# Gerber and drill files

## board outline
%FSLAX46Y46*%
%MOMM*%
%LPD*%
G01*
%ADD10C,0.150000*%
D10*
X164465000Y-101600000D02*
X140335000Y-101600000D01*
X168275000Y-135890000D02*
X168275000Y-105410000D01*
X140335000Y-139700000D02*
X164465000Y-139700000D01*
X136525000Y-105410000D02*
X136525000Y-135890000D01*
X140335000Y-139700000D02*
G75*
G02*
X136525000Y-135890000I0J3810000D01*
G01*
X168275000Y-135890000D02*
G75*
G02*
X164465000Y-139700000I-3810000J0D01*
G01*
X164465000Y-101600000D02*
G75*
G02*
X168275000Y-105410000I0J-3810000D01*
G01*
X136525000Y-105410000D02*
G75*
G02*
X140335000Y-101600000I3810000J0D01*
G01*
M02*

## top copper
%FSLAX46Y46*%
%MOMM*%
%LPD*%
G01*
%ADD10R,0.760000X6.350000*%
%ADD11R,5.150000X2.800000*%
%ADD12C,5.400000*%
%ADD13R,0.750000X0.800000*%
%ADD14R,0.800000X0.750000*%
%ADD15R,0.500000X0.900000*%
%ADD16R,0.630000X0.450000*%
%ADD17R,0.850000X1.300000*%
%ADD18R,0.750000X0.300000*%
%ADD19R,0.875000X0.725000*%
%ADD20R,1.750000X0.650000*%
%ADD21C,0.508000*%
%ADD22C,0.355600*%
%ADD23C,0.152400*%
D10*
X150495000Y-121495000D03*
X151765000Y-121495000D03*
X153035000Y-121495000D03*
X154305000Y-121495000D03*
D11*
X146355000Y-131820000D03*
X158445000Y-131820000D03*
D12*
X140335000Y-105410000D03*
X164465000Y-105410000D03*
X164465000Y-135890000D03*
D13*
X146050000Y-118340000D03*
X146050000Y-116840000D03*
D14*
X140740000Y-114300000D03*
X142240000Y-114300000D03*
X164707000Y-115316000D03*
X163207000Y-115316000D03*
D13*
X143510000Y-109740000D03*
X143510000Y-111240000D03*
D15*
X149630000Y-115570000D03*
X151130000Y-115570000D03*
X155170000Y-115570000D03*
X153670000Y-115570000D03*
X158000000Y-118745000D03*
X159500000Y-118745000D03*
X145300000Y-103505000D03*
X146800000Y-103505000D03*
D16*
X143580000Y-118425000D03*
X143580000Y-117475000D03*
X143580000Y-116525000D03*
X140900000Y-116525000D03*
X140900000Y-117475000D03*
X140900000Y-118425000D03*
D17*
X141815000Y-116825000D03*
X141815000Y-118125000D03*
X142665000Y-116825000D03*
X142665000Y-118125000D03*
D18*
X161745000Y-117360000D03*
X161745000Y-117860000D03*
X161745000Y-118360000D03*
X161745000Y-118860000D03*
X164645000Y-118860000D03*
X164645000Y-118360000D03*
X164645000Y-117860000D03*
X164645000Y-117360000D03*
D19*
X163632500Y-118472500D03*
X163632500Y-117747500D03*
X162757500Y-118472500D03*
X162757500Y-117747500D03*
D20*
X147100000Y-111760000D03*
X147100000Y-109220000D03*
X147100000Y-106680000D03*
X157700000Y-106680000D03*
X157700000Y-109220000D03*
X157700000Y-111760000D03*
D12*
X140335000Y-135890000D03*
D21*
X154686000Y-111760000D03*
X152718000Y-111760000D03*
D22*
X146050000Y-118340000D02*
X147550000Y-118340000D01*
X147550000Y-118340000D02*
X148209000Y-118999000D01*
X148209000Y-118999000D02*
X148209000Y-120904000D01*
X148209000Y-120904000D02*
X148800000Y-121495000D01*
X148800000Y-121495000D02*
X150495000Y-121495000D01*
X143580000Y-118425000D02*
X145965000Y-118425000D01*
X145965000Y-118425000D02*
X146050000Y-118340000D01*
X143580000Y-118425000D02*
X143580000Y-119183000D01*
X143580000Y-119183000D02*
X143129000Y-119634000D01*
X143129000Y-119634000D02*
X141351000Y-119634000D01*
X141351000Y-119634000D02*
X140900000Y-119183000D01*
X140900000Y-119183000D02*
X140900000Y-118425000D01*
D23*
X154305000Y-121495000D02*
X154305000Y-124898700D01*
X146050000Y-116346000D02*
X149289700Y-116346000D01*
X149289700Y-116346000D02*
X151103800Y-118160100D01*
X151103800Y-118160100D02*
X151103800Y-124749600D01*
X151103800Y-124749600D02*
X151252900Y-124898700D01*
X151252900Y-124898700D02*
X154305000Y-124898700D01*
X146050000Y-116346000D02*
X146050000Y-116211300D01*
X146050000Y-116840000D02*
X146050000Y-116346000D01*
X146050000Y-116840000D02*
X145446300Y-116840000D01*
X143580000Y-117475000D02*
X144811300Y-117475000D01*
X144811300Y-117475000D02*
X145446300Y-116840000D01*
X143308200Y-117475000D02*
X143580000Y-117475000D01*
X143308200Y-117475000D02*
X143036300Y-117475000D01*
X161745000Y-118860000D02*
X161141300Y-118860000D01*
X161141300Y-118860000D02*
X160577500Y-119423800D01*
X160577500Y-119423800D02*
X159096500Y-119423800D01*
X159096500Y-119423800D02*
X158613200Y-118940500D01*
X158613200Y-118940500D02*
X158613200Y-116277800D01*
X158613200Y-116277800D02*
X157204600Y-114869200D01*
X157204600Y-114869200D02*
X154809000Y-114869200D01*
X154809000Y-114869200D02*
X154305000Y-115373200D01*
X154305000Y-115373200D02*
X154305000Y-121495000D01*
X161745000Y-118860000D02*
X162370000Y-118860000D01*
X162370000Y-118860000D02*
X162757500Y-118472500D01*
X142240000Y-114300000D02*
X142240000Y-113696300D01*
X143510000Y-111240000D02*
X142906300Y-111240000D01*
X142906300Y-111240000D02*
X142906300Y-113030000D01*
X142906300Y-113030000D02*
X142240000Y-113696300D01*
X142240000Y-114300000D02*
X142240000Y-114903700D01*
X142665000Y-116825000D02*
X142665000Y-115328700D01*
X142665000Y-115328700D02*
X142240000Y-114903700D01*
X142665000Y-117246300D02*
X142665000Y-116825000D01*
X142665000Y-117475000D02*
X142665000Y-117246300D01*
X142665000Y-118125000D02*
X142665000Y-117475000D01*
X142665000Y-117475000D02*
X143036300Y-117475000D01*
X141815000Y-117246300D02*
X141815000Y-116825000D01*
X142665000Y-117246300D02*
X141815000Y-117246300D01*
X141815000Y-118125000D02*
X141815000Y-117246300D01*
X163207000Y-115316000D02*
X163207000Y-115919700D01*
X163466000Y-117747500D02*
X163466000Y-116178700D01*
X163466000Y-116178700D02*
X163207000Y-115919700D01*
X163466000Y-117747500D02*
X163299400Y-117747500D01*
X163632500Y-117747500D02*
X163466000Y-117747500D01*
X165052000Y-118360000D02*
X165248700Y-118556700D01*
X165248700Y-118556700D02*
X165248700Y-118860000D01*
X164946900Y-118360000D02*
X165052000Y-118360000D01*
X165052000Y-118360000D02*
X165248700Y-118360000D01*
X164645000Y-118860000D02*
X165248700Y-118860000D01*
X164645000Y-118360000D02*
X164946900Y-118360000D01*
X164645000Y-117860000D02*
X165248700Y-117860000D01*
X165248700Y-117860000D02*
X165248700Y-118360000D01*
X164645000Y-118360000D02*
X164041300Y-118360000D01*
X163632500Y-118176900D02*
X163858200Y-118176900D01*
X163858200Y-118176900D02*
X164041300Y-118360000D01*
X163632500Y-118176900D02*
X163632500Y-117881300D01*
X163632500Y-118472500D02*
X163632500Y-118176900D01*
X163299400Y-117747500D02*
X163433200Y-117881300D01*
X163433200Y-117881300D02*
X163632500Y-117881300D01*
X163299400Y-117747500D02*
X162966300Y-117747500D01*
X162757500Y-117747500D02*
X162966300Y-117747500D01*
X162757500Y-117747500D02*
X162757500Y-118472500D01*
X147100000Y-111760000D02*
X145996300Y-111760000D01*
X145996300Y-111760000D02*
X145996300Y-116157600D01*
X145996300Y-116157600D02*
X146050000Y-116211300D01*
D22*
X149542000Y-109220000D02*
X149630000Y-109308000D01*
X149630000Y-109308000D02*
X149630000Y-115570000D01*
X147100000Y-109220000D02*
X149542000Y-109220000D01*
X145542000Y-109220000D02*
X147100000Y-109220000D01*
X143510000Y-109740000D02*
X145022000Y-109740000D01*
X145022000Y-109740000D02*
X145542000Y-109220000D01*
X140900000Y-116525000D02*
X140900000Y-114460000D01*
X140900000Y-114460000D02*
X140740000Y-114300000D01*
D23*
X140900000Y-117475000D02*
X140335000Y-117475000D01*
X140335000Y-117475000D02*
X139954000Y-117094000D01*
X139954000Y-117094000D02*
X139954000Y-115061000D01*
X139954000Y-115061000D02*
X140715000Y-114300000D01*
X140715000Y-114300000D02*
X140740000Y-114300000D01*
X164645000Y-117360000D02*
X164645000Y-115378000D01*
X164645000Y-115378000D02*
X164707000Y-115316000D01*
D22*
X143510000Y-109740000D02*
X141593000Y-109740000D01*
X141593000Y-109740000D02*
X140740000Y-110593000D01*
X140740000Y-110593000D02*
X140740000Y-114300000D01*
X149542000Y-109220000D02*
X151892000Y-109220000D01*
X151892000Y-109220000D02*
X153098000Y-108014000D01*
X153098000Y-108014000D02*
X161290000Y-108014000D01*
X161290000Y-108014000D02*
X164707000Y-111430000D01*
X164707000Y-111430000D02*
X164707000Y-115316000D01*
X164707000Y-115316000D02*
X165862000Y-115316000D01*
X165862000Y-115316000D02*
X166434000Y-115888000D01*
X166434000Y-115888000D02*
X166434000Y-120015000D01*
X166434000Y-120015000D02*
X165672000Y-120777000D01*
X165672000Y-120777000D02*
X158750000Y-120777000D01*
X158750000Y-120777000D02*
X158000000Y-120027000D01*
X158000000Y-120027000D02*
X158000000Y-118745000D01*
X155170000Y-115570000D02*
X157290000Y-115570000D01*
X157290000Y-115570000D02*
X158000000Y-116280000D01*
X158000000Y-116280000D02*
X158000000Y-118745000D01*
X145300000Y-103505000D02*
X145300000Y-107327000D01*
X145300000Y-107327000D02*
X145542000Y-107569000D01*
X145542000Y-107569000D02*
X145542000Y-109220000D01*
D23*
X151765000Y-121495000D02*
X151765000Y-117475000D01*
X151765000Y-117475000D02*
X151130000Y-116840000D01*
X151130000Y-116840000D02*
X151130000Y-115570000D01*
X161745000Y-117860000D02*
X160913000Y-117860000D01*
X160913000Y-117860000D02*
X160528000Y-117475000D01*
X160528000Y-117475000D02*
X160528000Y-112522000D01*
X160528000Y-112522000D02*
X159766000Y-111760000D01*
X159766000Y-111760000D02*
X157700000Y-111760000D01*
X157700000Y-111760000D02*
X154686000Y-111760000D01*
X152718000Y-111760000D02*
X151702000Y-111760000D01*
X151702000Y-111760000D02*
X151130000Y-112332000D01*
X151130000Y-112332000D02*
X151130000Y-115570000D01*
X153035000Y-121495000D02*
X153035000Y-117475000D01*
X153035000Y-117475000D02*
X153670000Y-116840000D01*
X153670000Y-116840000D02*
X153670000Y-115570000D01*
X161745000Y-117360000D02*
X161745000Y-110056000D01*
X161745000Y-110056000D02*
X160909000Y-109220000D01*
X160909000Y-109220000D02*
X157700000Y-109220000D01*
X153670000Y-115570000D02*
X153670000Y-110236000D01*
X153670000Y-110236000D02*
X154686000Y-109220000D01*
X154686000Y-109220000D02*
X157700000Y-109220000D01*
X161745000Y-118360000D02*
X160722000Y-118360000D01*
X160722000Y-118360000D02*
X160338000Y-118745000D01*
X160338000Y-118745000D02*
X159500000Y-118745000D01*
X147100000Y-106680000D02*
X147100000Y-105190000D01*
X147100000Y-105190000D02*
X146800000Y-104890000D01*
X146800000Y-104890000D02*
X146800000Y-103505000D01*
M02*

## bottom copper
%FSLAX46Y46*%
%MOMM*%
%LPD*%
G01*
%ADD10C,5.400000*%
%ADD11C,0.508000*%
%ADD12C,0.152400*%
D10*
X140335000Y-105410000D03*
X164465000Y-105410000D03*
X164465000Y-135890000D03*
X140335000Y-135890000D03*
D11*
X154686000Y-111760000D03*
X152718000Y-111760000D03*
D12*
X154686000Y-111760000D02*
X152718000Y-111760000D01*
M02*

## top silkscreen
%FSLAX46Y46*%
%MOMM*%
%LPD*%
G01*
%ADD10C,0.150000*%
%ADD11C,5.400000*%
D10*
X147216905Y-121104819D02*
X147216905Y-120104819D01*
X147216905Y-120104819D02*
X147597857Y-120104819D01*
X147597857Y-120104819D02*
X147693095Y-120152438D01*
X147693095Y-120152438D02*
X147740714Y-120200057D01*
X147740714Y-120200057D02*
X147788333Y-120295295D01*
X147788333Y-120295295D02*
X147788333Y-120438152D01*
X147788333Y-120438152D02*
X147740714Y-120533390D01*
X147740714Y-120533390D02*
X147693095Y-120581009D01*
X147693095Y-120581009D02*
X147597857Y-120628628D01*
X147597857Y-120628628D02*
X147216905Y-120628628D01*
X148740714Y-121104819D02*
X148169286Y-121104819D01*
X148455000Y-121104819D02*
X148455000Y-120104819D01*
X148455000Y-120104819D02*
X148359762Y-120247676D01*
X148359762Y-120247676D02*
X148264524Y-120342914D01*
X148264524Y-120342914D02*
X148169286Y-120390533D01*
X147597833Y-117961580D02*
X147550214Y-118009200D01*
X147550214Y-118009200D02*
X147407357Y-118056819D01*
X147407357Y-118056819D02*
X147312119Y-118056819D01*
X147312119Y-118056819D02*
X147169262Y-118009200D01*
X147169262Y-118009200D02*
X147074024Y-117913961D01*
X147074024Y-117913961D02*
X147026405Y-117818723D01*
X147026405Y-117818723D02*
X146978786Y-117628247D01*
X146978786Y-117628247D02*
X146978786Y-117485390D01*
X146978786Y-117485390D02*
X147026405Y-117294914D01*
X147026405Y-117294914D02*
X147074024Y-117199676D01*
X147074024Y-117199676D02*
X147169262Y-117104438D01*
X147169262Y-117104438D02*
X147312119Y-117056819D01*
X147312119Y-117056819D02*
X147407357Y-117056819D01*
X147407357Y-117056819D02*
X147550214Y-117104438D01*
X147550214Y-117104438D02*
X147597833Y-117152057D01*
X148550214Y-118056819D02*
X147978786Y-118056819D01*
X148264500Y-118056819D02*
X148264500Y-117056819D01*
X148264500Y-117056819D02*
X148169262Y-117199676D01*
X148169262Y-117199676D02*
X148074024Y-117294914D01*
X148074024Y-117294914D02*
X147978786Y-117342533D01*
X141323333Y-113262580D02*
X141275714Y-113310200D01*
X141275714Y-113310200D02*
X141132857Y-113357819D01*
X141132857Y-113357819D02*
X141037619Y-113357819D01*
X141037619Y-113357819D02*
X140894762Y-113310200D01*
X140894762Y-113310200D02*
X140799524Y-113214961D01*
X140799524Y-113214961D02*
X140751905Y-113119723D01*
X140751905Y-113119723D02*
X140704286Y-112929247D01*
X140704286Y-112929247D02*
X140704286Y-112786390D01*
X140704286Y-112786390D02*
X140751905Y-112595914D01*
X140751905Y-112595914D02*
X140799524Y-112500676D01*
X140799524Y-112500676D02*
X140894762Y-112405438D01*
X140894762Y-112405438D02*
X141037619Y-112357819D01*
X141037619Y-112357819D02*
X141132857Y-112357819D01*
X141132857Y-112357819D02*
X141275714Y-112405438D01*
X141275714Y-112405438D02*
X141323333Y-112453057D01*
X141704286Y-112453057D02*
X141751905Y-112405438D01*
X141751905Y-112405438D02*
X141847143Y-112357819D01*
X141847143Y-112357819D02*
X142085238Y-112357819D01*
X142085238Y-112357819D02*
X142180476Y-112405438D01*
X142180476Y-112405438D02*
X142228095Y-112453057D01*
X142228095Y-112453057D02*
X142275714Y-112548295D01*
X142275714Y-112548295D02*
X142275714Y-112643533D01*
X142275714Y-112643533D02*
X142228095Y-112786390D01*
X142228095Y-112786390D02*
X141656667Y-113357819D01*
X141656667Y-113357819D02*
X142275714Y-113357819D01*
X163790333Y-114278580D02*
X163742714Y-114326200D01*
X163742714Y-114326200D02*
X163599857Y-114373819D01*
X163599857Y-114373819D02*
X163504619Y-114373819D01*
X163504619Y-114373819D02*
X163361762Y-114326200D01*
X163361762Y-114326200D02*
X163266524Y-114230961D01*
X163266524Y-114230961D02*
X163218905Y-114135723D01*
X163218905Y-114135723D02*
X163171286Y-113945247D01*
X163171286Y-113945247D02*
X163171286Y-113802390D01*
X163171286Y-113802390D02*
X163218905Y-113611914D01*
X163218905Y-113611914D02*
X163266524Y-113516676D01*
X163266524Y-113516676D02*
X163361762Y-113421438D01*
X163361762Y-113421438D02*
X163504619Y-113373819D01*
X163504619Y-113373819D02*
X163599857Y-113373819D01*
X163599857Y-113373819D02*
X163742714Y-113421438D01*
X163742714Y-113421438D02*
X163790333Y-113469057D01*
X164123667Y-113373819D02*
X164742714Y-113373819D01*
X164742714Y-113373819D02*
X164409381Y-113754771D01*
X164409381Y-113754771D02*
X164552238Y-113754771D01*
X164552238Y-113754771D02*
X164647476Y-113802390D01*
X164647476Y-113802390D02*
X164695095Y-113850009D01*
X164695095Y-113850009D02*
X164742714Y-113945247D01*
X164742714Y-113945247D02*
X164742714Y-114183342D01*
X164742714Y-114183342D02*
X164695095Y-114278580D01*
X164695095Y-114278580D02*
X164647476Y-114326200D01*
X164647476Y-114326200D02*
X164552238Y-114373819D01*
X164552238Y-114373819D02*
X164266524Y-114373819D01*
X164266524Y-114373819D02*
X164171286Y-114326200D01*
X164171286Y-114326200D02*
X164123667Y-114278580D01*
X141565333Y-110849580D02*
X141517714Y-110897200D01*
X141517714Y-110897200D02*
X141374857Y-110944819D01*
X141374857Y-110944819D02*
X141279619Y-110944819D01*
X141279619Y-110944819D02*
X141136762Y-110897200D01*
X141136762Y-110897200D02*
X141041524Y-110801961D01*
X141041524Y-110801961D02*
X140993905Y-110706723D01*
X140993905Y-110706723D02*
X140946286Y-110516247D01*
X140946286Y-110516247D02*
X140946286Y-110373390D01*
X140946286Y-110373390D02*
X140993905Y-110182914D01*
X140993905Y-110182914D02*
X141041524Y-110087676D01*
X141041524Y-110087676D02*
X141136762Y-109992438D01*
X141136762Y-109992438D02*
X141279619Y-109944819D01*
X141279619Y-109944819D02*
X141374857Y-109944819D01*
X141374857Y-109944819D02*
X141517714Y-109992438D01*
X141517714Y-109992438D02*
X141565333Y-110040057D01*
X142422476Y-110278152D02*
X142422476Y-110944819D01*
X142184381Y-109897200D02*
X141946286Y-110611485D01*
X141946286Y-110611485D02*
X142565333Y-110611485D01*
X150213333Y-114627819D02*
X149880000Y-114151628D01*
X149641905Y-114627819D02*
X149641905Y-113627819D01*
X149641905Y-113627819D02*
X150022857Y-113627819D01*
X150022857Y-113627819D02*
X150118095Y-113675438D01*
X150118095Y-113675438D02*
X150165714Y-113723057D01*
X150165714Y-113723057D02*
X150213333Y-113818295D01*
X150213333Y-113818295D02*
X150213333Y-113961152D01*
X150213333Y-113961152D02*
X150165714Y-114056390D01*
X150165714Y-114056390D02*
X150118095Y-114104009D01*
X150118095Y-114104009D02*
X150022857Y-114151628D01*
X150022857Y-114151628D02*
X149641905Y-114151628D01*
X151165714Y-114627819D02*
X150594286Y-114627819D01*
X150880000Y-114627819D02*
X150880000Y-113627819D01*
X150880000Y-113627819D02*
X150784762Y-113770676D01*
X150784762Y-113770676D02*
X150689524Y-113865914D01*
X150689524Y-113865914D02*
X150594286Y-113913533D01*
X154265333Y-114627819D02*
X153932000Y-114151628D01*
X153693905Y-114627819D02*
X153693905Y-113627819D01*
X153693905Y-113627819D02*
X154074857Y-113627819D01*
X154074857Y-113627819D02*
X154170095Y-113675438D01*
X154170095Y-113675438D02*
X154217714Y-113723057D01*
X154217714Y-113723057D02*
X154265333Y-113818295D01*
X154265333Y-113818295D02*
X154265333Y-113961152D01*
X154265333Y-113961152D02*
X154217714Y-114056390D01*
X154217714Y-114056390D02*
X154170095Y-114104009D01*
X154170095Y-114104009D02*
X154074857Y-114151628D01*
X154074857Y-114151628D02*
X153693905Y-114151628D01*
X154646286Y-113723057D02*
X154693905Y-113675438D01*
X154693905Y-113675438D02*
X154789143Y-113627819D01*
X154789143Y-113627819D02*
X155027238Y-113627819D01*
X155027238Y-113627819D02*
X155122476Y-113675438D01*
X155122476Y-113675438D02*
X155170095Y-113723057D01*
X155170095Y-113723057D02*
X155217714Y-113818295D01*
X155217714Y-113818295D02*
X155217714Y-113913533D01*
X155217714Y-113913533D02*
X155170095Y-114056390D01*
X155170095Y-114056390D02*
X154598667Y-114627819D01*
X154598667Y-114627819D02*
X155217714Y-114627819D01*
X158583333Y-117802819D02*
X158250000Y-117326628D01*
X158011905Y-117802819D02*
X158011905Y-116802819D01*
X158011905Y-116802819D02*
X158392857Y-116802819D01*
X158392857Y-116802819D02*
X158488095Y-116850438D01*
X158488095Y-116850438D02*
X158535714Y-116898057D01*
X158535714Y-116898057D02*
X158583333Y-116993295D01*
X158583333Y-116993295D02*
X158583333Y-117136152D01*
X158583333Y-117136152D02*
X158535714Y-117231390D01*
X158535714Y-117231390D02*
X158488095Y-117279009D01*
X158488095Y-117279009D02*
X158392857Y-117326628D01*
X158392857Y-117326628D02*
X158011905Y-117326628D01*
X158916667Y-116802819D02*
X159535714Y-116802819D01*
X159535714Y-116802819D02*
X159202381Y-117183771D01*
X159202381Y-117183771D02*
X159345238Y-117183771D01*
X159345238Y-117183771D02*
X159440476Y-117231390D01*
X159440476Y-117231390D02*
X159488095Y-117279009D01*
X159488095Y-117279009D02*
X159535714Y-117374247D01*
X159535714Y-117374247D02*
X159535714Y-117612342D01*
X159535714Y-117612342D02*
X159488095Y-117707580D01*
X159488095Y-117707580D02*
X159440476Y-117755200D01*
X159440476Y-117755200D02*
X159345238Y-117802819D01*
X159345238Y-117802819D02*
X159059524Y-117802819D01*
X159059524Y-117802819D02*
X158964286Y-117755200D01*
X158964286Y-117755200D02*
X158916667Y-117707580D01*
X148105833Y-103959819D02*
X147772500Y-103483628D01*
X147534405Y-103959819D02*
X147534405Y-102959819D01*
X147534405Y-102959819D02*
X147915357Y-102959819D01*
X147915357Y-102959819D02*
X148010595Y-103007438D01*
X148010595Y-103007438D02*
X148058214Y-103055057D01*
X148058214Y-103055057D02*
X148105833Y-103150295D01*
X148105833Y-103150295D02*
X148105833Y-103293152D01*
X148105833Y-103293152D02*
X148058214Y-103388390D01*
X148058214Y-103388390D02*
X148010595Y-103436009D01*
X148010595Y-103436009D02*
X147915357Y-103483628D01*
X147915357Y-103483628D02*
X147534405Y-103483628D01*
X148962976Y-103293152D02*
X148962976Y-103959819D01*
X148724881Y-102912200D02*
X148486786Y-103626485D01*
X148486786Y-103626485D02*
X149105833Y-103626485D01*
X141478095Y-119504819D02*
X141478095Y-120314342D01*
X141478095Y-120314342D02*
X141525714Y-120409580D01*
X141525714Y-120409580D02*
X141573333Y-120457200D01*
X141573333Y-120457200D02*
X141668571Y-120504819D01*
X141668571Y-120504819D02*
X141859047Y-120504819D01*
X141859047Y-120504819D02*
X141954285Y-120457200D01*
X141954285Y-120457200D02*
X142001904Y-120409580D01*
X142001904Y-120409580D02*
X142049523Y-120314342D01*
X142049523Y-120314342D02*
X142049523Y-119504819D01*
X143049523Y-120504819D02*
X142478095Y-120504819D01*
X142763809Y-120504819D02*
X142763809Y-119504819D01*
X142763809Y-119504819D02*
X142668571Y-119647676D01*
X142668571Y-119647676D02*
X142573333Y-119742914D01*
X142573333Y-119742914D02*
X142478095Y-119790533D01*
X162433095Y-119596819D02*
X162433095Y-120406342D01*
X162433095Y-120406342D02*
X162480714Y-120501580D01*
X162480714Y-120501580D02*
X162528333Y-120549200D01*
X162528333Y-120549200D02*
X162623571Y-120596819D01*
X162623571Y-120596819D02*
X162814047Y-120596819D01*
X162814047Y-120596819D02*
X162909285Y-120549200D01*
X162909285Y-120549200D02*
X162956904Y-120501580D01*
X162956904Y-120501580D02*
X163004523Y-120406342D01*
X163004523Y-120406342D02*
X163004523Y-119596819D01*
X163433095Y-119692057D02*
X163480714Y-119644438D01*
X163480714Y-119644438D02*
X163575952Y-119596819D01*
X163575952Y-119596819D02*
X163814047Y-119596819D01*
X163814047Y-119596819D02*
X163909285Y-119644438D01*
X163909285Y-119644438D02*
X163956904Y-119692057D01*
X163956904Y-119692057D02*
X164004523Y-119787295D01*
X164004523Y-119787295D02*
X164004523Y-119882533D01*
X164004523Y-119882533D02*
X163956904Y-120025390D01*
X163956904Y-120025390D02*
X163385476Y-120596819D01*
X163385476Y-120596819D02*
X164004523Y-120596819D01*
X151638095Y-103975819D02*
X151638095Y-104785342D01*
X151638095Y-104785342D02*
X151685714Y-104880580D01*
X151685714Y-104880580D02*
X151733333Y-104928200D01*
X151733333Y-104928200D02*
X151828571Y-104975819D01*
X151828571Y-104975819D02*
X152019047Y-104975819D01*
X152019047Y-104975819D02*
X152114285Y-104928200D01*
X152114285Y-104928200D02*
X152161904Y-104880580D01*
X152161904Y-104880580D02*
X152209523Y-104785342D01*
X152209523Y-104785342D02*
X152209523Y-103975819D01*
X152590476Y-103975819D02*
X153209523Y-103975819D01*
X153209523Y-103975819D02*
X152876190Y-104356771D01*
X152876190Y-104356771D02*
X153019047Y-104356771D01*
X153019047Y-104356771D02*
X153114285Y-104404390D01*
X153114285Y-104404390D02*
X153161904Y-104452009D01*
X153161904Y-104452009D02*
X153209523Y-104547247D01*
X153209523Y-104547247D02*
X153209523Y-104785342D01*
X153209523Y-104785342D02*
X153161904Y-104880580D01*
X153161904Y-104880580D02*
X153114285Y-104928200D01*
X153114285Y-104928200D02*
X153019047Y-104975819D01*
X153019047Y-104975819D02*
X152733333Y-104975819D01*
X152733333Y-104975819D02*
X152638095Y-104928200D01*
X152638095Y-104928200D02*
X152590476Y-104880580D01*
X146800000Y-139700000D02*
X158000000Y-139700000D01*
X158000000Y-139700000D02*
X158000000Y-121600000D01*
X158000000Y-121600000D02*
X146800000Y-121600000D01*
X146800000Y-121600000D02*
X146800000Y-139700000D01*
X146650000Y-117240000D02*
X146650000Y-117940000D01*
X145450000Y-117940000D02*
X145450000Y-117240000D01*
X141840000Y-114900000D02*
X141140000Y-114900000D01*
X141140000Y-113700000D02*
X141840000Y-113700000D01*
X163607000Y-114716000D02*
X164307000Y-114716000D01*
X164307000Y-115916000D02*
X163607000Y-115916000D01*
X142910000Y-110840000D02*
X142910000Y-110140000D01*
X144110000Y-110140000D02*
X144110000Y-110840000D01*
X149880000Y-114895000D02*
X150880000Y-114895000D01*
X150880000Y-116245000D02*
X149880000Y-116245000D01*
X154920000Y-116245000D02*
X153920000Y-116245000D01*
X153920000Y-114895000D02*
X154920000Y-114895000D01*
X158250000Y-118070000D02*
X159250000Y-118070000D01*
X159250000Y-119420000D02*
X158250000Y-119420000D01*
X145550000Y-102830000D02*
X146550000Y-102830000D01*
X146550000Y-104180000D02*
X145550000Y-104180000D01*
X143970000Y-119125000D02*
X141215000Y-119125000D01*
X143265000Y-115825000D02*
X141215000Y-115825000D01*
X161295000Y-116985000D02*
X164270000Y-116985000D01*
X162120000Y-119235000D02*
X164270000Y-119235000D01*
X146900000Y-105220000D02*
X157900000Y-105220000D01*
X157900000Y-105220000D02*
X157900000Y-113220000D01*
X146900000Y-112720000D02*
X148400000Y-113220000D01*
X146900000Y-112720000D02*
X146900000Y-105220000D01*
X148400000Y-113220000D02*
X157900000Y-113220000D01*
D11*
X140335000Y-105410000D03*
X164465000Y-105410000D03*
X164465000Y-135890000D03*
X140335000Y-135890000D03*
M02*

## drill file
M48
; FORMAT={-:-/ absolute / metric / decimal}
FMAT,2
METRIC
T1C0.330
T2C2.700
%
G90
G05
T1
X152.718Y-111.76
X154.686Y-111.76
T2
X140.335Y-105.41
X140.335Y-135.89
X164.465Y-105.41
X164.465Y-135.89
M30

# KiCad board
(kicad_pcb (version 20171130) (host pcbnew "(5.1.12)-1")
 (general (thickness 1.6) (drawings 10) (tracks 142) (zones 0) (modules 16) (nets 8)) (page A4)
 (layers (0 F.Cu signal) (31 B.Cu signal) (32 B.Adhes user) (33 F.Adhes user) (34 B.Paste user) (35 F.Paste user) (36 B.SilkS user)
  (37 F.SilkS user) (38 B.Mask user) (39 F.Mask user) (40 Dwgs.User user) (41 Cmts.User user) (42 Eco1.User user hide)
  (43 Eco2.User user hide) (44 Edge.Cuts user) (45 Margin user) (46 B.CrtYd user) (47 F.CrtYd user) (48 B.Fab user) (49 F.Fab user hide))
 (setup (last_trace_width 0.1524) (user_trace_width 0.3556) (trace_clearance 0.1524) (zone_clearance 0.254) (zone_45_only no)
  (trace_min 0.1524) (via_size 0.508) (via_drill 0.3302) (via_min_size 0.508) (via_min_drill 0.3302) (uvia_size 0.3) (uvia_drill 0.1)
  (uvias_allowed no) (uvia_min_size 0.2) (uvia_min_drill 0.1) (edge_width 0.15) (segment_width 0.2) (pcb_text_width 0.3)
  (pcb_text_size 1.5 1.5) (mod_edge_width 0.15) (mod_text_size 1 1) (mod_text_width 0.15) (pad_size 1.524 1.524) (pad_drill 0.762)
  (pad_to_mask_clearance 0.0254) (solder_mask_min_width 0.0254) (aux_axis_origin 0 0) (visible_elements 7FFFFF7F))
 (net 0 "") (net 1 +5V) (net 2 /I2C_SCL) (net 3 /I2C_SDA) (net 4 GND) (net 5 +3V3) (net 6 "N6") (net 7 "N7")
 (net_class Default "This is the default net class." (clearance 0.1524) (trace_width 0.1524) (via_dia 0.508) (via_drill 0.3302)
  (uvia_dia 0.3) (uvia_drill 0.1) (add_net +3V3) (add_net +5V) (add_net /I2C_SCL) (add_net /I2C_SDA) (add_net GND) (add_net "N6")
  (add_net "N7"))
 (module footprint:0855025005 (layer F.Cu) (at 152.4 139.7)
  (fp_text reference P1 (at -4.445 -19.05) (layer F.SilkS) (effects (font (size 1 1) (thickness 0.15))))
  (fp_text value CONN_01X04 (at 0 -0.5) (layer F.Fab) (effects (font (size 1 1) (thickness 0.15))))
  (fp_line (start -5.6 0) (end 5.6 0) (layer F.SilkS) (width 0.15))
  (fp_line (start 5.6 0) (end 5.6 -18.1) (layer F.SilkS) (width 0.15))
  (fp_line (start 5.6 -18.1) (end -5.6 -18.1) (layer F.SilkS) (width 0.15))
  (fp_line (start -5.6 -18.1) (end -5.6 0) (layer F.SilkS) (width 0.15))
  (pad 1 smd rect (at -1.905 -18.205) (size 0.76 6.35) (layers F.Cu F.Paste F.Mask) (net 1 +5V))
  (pad 2 smd rect (at -0.635 -18.205) (size 0.76 6.35) (layers F.Cu F.Paste F.Mask) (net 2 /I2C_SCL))
  (pad 3 smd rect (at 0.635 -18.205) (size 0.76 6.35) (layers F.Cu F.Paste F.Mask) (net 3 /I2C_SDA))
  (pad 4 smd rect (at 1.905 -18.205) (size 0.76 6.35) (layers F.Cu F.Paste F.Mask) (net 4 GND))
  (pad 5 smd rect (at -6.045 -7.88) (size 5.15 2.8) (layers F.Cu F.Paste F.Mask))
  (pad 5 smd rect (at 6.045 -7.88) (size 5.15 2.8) (layers F.Cu F.Paste F.Mask)))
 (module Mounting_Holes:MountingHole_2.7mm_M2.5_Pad (layer F.Cu) (at 140.335 105.41)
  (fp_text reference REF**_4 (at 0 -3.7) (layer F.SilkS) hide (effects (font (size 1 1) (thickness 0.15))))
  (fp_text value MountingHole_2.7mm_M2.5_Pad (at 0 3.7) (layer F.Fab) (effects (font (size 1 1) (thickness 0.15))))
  (pad 1 thru_hole circle (at 0 0) (size 5.4 5.4) (drill 2.7) (layers *.Cu *.Mask F.SilkS)))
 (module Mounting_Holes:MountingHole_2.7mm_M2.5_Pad (layer F.Cu) (at 164.465 105.41)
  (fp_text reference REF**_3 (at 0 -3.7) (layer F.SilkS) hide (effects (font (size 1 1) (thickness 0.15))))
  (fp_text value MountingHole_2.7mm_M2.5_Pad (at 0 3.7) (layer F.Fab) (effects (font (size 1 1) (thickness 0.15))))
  (pad 1 thru_hole circle (at 0 0) (size 5.4 5.4) (drill 2.7) (layers *.Cu *.Mask F.SilkS)))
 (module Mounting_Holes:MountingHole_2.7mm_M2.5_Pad (layer F.Cu) (at 164.465 135.89)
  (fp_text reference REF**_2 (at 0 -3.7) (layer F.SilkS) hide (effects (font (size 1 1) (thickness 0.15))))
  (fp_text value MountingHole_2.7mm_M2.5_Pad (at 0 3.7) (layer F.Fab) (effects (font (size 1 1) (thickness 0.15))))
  (pad 1 thru_hole circle (at 0 0) (size 5.4 5.4) (drill 2.7) (layers *.Cu *.Mask F.SilkS)))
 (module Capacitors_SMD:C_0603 (layer F.Cu) (at 146.05 117.59 90)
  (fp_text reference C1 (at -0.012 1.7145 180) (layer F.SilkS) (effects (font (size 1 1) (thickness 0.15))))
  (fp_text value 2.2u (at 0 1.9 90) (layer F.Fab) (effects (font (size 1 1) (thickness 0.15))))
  (fp_line (start 0.35 0.6) (end -0.35 0.6) (layer F.SilkS) (width 0.15))
  (fp_line (start -0.35 -0.6) (end 0.35 -0.6) (layer F.SilkS) (width 0.15))
  (pad 1 smd rect (at -0.75 0 90) (size 0.8 0.75) (layers F.Cu F.Paste F.Mask) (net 1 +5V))
  (pad 2 smd rect (at 0.75 0 90) (size 0.8 0.75) (layers F.Cu F.Paste F.Mask) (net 4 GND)))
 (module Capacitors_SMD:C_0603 (layer F.Cu) (at 141.49 114.3)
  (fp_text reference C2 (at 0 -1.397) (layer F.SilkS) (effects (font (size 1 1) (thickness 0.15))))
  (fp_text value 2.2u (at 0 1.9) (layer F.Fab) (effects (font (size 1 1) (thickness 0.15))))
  (fp_line (start 0.35 0.6) (end -0.35 0.6) (layer F.SilkS) (width 0.15))
  (fp_line (start -0.35 -0.6) (end 0.35 -0.6) (layer F.SilkS) (width 0.15))
  (pad 1 smd rect (at -0.75 0) (size 0.8 0.75) (layers F.Cu F.Paste F.Mask) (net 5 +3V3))
  (pad 2 smd rect (at 0.75 0) (size 0.8 0.75) (layers F.Cu F.Paste F.Mask) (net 4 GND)))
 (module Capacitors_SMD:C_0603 (layer F.Cu) (at 163.957 115.316 180)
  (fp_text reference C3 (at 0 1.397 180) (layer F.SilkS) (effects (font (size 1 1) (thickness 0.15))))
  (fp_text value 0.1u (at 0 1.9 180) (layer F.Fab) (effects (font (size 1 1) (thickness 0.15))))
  (fp_line (start 0.35 0.6) (end -0.35 0.6) (layer F.SilkS) (width 0.15))
  (fp_line (start -0.35 -0.6) (end 0.35 -0.6) (layer F.SilkS) (width 0.15))
  (pad 1 smd rect (at -0.75 0 180) (size 0.8 0.75) (layers F.Cu F.Paste F.Mask) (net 5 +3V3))
  (pad 2 smd rect (at 0.75 0 180) (size 0.8 0.75) (layers F.Cu F.Paste F.Mask) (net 4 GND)))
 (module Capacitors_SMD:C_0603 (layer F.Cu) (at 143.51 110.49 270)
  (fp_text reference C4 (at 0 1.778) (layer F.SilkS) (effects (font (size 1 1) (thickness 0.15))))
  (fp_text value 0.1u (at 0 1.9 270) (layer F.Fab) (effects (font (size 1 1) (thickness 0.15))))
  (fp_line (start 0.35 0.6) (end -0.35 0.6) (layer F.SilkS) (width 0.15))
  (fp_line (start -0.35 -0.6) (end 0.35 -0.6) (layer F.SilkS) (width 0.15))
  (pad 1 smd rect (at -0.75 0 270) (size 0.8 0.75) (layers F.Cu F.Paste F.Mask) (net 5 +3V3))
  (pad 2 smd rect (at 0.75 0 270) (size 0.8 0.75) (layers F.Cu F.Paste F.Mask) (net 4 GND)))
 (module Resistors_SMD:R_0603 (layer F.Cu) (at 150.38 115.57)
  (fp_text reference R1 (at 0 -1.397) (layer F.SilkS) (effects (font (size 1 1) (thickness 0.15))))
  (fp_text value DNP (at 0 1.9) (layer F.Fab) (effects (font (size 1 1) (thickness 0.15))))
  (fp_line (start -0.5 -0.675) (end 0.5 -0.675) (layer F.SilkS) (width 0.15))
  (fp_line (start 0.5 0.675) (end -0.5 0.675) (layer F.SilkS) (width 0.15))
  (pad 1 smd rect (at -0.75 0) (size 0.5 0.9) (layers F.Cu F.Paste F.Mask) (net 5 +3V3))
  (pad 2 smd rect (at 0.75 0) (size 0.5 0.9) (layers F.Cu F.Paste F.Mask) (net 2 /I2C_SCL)))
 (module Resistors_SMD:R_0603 (layer F.Cu) (at 154.42 115.57 180)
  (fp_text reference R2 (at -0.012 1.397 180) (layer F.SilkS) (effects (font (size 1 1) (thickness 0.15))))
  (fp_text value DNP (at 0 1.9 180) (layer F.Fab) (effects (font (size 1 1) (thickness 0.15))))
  (fp_line (start -0.5 -0.675) (end 0.5 -0.675) (layer F.SilkS) (width 0.15))
  (fp_line (start 0.5 0.675) (end -0.5 0.675) (layer F.SilkS) (width 0.15))
  (pad 1 smd rect (at -0.75 0 180) (size 0.5 0.9) (layers F.Cu F.Paste F.Mask) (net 5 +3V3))
  (pad 2 smd rect (at 0.75 0 180) (size 0.5 0.9) (layers F.Cu F.Paste F.Mask) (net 3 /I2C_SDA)))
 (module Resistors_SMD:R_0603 (layer F.Cu) (at 158.75 118.745)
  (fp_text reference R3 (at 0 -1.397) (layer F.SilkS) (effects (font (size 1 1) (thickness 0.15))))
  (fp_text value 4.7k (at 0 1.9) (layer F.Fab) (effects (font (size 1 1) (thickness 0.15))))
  (fp_line (start -0.5 -0.675) (end 0.5 -0.675) (layer F.SilkS) (width 0.15))
  (fp_line (start 0.5 0.675) (end -0.5 0.675) (layer F.SilkS) (width 0.15))
  (pad 1 smd rect (at -0.75 0) (size 0.5 0.9) (layers F.Cu F.Paste F.Mask) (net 5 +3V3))
  (pad 2 smd rect (at 0.75 0) (size 0.5 0.9) (layers F.Cu F.Paste F.Mask) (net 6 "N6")))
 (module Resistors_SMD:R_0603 (layer F.Cu) (at 146.05 103.505)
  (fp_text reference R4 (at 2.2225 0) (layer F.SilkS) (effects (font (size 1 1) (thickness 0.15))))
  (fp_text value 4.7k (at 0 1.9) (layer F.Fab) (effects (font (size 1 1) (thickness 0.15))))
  (fp_line (start -0.5 -0.675) (end 0.5 -0.675) (layer F.SilkS) (width 0.15))
  (fp_line (start 0.5 0.675) (end -0.5 0.675) (layer F.SilkS) (width 0.15))
  (pad 1 smd rect (at -0.75 0) (size 0.5 0.9) (layers F.Cu F.Paste F.Mask) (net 5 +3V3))
  (pad 2 smd rect (at 0.75 0) (size 0.5 0.9) (layers F.Cu F.Paste F.Mask) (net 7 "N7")))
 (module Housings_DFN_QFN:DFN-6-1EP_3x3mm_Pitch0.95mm (layer F.Cu) (at 142.24 117.475 180)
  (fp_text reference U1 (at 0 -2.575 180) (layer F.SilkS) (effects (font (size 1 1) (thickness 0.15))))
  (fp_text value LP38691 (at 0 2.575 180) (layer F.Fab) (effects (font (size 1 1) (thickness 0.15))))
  (fp_line (start -1.73 -1.65) (end 1.025 -1.65) (layer F.SilkS) (width 0.15))
  (fp_line (start -1.025 1.65) (end 1.025 1.65) (layer F.SilkS) (width 0.15))
  (pad 1 smd rect (at -1.34 -0.95 180) (size 0.63 0.45) (layers F.Cu F.Paste F.Mask) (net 1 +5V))
  (pad 2 smd rect (at -1.34 0 180) (size 0.63 0.45) (layers F.Cu F.Paste F.Mask) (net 4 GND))
  (pad 3 smd rect (at -1.34 0.95 180) (size 0.63 0.45) (layers F.Cu F.Paste F.Mask))
  (pad 4 smd rect (at 1.34 0.95 180) (size 0.63 0.45) (layers F.Cu F.Paste F.Mask) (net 5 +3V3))
  (pad 5 smd rect (at 1.34 0 180) (size 0.63 0.45) (layers F.Cu F.Paste F.Mask) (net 5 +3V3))
  (pad 6 smd rect (at 1.34 -0.95 180) (size 0.63 0.45) (layers F.Cu F.Paste F.Mask) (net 1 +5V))
  (pad 7 smd rect (at 0.425 0.65 180) (size 0.85 1.3) (layers F.Cu F.Paste F.Mask) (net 4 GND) (solder_paste_margin_ratio -0.2))
  (pad 7 smd rect (at 0.425 -0.65 180) (size 0.85 1.3) (layers F.Cu F.Paste F.Mask) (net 4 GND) (solder_paste_margin_ratio -0.2))
  (pad 7 smd rect (at -0.425 0.65 180) (size 0.85 1.3) (layers F.Cu F.Paste F.Mask) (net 4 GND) (solder_paste_margin_ratio -0.2))
  (pad 7 smd rect (at -0.425 -0.65 180) (size 0.85 1.3) (layers F.Cu F.Paste F.Mask) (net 4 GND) (solder_paste_margin_ratio -0.2)))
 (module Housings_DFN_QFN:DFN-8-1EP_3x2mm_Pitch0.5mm (layer F.Cu) (at 163.195 118.11)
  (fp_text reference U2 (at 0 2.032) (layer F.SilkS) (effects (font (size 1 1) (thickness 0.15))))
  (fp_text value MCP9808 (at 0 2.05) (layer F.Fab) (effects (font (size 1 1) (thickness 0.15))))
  (fp_line (start -1.9 -1.125) (end 1.075 -1.125) (layer F.SilkS) (width 0.15))
  (fp_line (start -1.075 1.125) (end 1.075 1.125) (layer F.SilkS) (width 0.15))
  (pad 1 smd rect (at -1.45 -0.75) (size 0.75 0.3) (layers F.Cu F.Paste F.Mask) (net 3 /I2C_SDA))
  (pad 2 smd rect (at -1.45 -0.25) (size 0.75 0.3) (layers F.Cu F.Paste F.Mask) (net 2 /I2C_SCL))
  (pad 3 smd rect (at -1.45 0.25) (size 0.75 0.3) (layers F.Cu F.Paste F.Mask) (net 6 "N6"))
  (pad 4 smd rect (at -1.45 0.75) (size 0.75 0.3) (layers F.Cu F.Paste F.Mask) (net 4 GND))
  (pad 5 smd rect (at 1.45 0.75) (size 0.75 0.3) (layers F.Cu F.Paste F.Mask) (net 4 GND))
  (pad 6 smd rect (at 1.45 0.25) (size 0.75 0.3) (layers F.Cu F.Paste F.Mask) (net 4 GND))
  (pad 7 smd rect (at 1.45 -0.25) (size 0.75 0.3) (layers F.Cu F.Paste F.Mask) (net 4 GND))
  (pad 8 smd rect (at 1.45 -0.75) (size 0.75 0.3) (layers F.Cu F.Paste F.Mask) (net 5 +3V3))
  (pad 9 smd rect (at 0.4375 0.3625) (size 0.875 0.725) (layers F.Cu F.Paste F.Mask) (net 4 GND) (solder_paste_margin_ratio -0.2))
  (pad 9 smd rect (at 0.4375 -0.3625) (size 0.875 0.725) (layers F.Cu F.Paste F.Mask) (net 4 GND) (solder_paste_margin_ratio -0.2))
  (pad 9 smd rect (at -0.4375 0.3625) (size 0.875 0.725) (layers F.Cu F.Paste F.Mask) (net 4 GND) (solder_paste_margin_ratio -0.2))
  (pad 9 smd rect (at -0.4375 -0.3625) (size 0.875 0.725) (layers F.Cu F.Paste F.Mask) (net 4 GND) (solder_paste_margin_ratio -0.2)))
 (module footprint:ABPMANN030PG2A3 (layer F.Cu) (at 152.4 109.22)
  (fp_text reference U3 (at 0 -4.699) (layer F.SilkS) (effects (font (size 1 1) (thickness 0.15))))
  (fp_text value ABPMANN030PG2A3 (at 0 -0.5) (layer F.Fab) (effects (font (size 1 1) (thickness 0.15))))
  (fp_line (start -5.5 -4) (end 5.5 -4) (layer F.SilkS) (width 0.15))
  (fp_line (start 5.5 -4) (end 5.5 4) (layer F.SilkS) (width 0.15))
  (fp_line (start -5.5 3.5) (end -4 4) (layer F.SilkS) (width 0.15))
  (fp_line (start -5.5 3.5) (end -5.5 -4) (layer F.SilkS) (width 0.15))
  (fp_line (start -4 4) (end 5.5 4) (layer F.SilkS) (width 0.15))
  (pad 1 smd rect (at -5.3 2.54) (size 1.75 0.65) (layers F.Cu F.Paste F.Mask) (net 4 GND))
  (pad 2 smd rect (at -5.3 0) (size 1.75 0.65) (layers F.Cu F.Paste F.Mask) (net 5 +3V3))
  (pad 3 smd rect (at -5.3 -2.54) (size 1.75 0.65) (layers F.Cu F.Paste F.Mask) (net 7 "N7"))
  (pad 4 smd rect (at 5.3 -2.54) (size 1.75 0.65) (layers F.Cu F.Paste F.Mask))
  (pad 5 smd rect (at 5.3 0) (size 1.75 0.65) (layers F.Cu F.Paste F.Mask) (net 3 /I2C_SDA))
  (pad 6 smd rect (at 5.3 2.54) (size 1.75 0.65) (layers F.Cu F.Paste F.Mask) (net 2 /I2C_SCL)))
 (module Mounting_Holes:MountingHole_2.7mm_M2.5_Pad (layer F.Cu) (at 140.335 135.89)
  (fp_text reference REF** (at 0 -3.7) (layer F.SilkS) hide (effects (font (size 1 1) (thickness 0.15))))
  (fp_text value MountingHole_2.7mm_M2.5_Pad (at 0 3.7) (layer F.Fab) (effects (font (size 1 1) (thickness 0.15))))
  (pad 1 thru_hole circle (at 0 0) (size 5.4 5.4) (drill 2.7) (layers *.Cu *.Mask F.SilkS)))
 (gr_line (start 164.465 101.6) (end 140.335 101.6) (layer Edge.Cuts) (width 0.15))
 (gr_line (start 168.275 135.89) (end 168.275 105.41) (layer Edge.Cuts) (width 0.15))
 (gr_line (start 140.335 139.7) (end 164.465 139.7) (layer Edge.Cuts) (width 0.15))
 (gr_line (start 136.525 105.41) (end 136.525 135.89) (layer Edge.Cuts) (width 0.15))
 (gr_arc (start 140.335 135.89) (end 140.335 139.7) (angle 90) (layer Edge.Cuts) (width 0.15))
 (gr_arc (start 164.465 135.89) (end 168.275 135.89) (angle 90) (layer Edge.Cuts) (width 0.15))
 (gr_arc (start 164.465 105.41) (end 164.465 101.6) (angle 90) (layer Edge.Cuts) (width 0.15))
 (gr_arc (start 140.335 105.41) (end 136.525 105.41) (angle 90) (layer Edge.Cuts) (width 0.15))
 (segment (start 146.05 118.34) (end 147.55 118.34) (width 0.3556) (layer F.Cu) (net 1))
 (segment (start 147.55 118.34) (end 148.209 118.999) (width 0.3556) (layer F.Cu) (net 1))
 (segment (start 148.209 118.999) (end 148.209 120.904) (width 0.3556) (layer F.Cu) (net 1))
 (segment (start 148.209 120.904) (end 148.8 121.495) (width 0.3556) (layer F.Cu) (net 1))
 (segment (start 148.8 121.495) (end 150.495 121.495) (width 0.3556) (layer F.Cu) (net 1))
 (segment (start 143.58 118.425) (end 145.965 118.425) (width 0.3556) (layer F.Cu) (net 1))
 (segment (start 145.965 118.425) (end 146.05 118.34) (width 0.3556) (layer F.Cu) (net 1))
 (segment (start 143.58 118.425) (end 143.58 119.183) (width 0.3556) (layer F.Cu) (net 1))
 (segment (start 143.58 119.183) (end 143.129 119.634) (width 0.3556) (layer F.Cu) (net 1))
 (segment (start 143.129 119.634) (end 141.351 119.634) (width 0.3556) (layer F.Cu) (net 1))
 (segment (start 141.351 119.634) (end 140.9 119.183) (width 0.3556) (layer F.Cu) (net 1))
 (segment (start 140.9 119.183) (end 140.9 118.425) (width 0.3556) (layer F.Cu) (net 1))
 (segment (start 154.305 121.495) (end 154.305 124.8987) (width 0.1524) (layer F.Cu) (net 4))
 (segment (start 146.05 116.346) (end 149.2897 116.346) (width 0.1524) (layer F.Cu) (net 4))
 (segment (start 149.2897 116.346) (end 151.1038 118.1601) (width 0.1524) (layer F.Cu) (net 4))
 (segment (start 151.1038 118.1601) (end 151.1038 124.7496) (width 0.1524) (layer F.Cu) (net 4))
 (segment (start 151.1038 124.7496) (end 151.2529 124.8987) (width 0.1524) (layer F.Cu) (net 4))
 (segment (start 151.2529 124.8987) (end 154.305 124.8987) (width 0.1524) (layer F.Cu) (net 4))
 (segment (start 146.05 116.346) (end 146.05 116.2113) (width 0.1524) (layer F.Cu) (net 4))
 (segment (start 146.05 116.84) (end 146.05 116.346) (width 0.1524) (layer F.Cu) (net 4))
 (segment (start 146.05 116.84) (end 145.4463 116.84) (width 0.1524) (layer F.Cu) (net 4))
 (segment (start 143.58 117.475) (end 144.8113 117.475) (width 0.1524) (layer F.Cu) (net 4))
 (segment (start 144.8113 117.475) (end 145.4463 116.84) (width 0.1524) (layer F.Cu) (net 4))
 (segment (start 143.3082 117.475) (end 143.58 117.475) (width 0.1524) (layer F.Cu) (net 4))
 (segment (start 143.3082 117.475) (end 143.0363 117.475) (width 0.1524) (layer F.Cu) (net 4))
 (segment (start 161.745 118.86) (end 161.1413 118.86) (width 0.1524) (layer F.Cu) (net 4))
 (segment (start 161.1413 118.86) (end 160.5775 119.4238) (width 0.1524) (layer F.Cu) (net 4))
 (segment (start 160.5775 119.4238) (end 159.0965 119.4238) (width 0.1524) (layer F.Cu) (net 4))
 (segment (start 159.0965 119.4238) (end 158.6132 118.9405) (width 0.1524) (layer F.Cu) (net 4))
 (segment (start 158.6132 118.9405) (end 158.6132 116.2778) (width 0.1524) (layer F.Cu) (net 4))
 (segment (start 158.6132 116.2778) (end 157.2046 114.8692) (width 0.1524) (layer F.Cu) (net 4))
 (segment (start 157.2046 114.8692) (end 154.809 114.8692) (width 0.1524) (layer F.Cu) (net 4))
 (segment (start 154.809 114.8692) (end 154.305 115.3732) (width 0.1524) (layer F.Cu) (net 4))
 (segment (start 154.305 115.3732) (end 154.305 121.495) (width 0.1524) (layer F.Cu) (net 4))
 (segment (start 161.745 118.86) (end 162.37 118.86) (width 0.1524) (layer F.Cu) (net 4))
 (segment (start 162.37 118.86) (end 162.7575 118.4725) (width 0.1524) (layer F.Cu) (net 4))
 (segment (start 142.24 114.3) (end 142.24 113.6963) (width 0.1524) (layer F.Cu) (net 4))
 (segment (start 143.51 111.24) (end 142.9063 111.24) (width 0.1524) (layer F.Cu) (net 4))
 (segment (start 142.9063 111.24) (end 142.9063 113.03) (width 0.1524) (layer F.Cu) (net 4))
 (segment (start 142.9063 113.03) (end 142.24 113.6963) (width 0.1524) (layer F.Cu) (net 4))
 (segment (start 142.24 114.3) (end 142.24 114.9037) (width 0.1524) (layer F.Cu) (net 4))
 (segment (start 142.665 116.825) (end 142.665 115.3287) (width 0.1524) (layer F.Cu) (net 4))
 (segment (start 142.665 115.3287) (end 142.24 114.9037) (width 0.1524) (layer F.Cu) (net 4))
 (segment (start 142.665 117.2463) (end 142.665 116.825) (width 0.1524) (layer F.Cu) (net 4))
 (segment (start 142.665 117.475) (end 142.665 117.2463) (width 0.1524) (layer F.Cu) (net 4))
 (segment (start 142.665 118.125) (end 142.665 117.475) (width 0.1524) (layer F.Cu) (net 4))
 (segment (start 142.665 117.475) (end 143.0363 117.475) (width 0.1524) (layer F.Cu) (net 4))
 (segment (start 141.815 117.2463) (end 141.815 116.825) (width 0.1524) (layer F.Cu) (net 4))
 (segment (start 142.665 117.2463) (end 141.815 117.2463) (width 0.1524) (layer F.Cu) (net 4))
 (segment (start 141.815 118.125) (end 141.815 117.2463) (width 0.1524) (layer F.Cu) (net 4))
 (segment (start 163.207 115.316) (end 163.207 115.9197) (width 0.1524) (layer F.Cu) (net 4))
 (segment (start 163.466 117.7475) (end 163.466 116.1787) (width 0.1524) (layer F.Cu) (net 4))
 (segment (start 163.466 116.1787) (end 163.207 115.9197) (width 0.1524) (layer F.Cu) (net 4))
 (segment (start 163.466 117.7475) (end 163.2994 117.7475) (width 0.1524) (layer F.Cu) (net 4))
 (segment (start 163.6325 117.7475) (end 163.466 117.7475) (width 0.1524) (layer F.Cu) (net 4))
 (segment (start 165.052 118.36) (end 165.2487 118.5567) (width 0.1524) (layer F.Cu) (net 4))
 (segment (start 165.2487 118.5567) (end 165.2487 118.86) (width 0.1524) (layer F.Cu) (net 4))
 (segment (start 164.9469 118.36) (end 165.052 118.36) (width 0.1524) (layer F.Cu) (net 4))
 (segment (start 165.052 118.36) (end 165.2487 118.36) (width 0.1524) (layer F.Cu) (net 4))
 (segment (start 164.645 118.86) (end 165.2487 118.86) (width 0.1524) (layer F.Cu) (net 4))
 (segment (start 164.645 118.36) (end 164.9469 118.36) (width 0.1524) (layer F.Cu) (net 4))
 (segment (start 164.645 117.86) (end 165.2487 117.86) (width 0.1524) (layer F.Cu) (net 4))
 (segment (start 165.2487 117.86) (end 165.2487 118.36) (width 0.1524) (layer F.Cu) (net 4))
 (segment (start 164.645 118.36) (end 164.0413 118.36) (width 0.1524) (layer F.Cu) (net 4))
 (segment (start 163.6325 118.1769) (end 163.8582 118.1769) (width 0.1524) (layer F.Cu) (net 4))
 (segment (start 163.8582 118.1769) (end 164.0413 118.36) (width 0.1524) (layer F.Cu) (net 4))
 (segment (start 163.6325 118.1769) (end 163.6325 117.8813) (width 0.1524) (layer F.Cu) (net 4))
 (segment (start 163.6325 118.4725) (end 163.6325 118.1769) (width 0.1524) (layer F.Cu) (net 4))
 (segment (start 163.2994 117.7475) (end 163.4332 117.8813) (width 0.1524) (layer F.Cu) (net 4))
 (segment (start 163.4332 117.8813) (end 163.6325 117.8813) (width 0.1524) (layer F.Cu) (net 4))
 (segment (start 163.2994 117.7475) (end 162.9663 117.7475) (width 0.1524) (layer F.Cu) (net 4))
 (segment (start 162.7575 117.7475) (end 162.9663 117.7475) (width 0.1524) (layer F.Cu) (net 4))
 (segment (start 162.7575 117.7475) (end 162.7575 118.4725) (width 0.1524) (layer F.Cu) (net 4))
 (segment (start 147.1 111.76) (end 145.9963 111.76) (width 0.1524) (layer F.Cu) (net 4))
 (segment (start 145.9963 111.76) (end 145.9963 116.1576) (width 0.1524) (layer F.Cu) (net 4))
 (segment (start 145.9963 116.1576) (end 146.05 116.2113) (width 0.1524) (layer F.Cu) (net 4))
 (segment (start 149.542 109.22) (end 149.63 109.308) (width 0.3556) (layer F.Cu) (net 5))
 (segment (start 149.63 109.308) (end 149.63 115.57) (width 0.3556) (layer F.Cu) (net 5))
 (segment (start 147.1 109.22) (end 149.542 109.22) (width 0.3556) (layer F.Cu) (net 5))
 (segment (start 145.542 109.22) (end 147.1 109.22) (width 0.3556) (layer F.Cu) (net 5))
 (segment (start 143.51 109.74) (end 145.022 109.74) (width 0.3556) (layer F.Cu) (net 5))
 (segment (start 145.022 109.74) (end 145.542 109.22) (width 0.3556) (layer F.Cu) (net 5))
 (segment (start 140.9 116.525) (end 140.9 114.46) (width 0.3556) (layer F.Cu) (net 5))
 (segment (start 140.9 114.46) (end 140.74 114.3) (width 0.3556) (layer F.Cu) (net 5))
 (segment (start 140.9 117.475) (end 140.335 117.475) (width 0.1524) (layer F.Cu) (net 5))
 (segment (start 140.335 117.475) (end 139.954 117.094) (width 0.1524) (layer F.Cu) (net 5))
 (segment (start 139.954 117.094) (end 139.954 115.061) (width 0.1524) (layer F.Cu) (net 5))
 (segment (start 139.954 115.061) (end 140.715 114.3) (width 0.1524) (layer F.Cu) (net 5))
 (segment (start 140.715 114.3) (end 140.74 114.3) (width 0.1524) (layer F.Cu) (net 5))
 (segment (start 164.645 117.36) (end 164.645 115.378) (width 0.1524) (layer F.Cu) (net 5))
 (segment (start 164.645 115.378) (end 164.707 115.316) (width 0.1524) (layer F.Cu) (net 5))
 (segment (start 143.51 109.74) (end 141.593 109.74) (width 0.3556) (layer F.Cu) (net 5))
 (segment (start 141.593 109.74) (end 140.74 110.593) (width 0.3556) (layer F.Cu) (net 5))
 (segment (start 140.74 110.593) (end 140.74 114.3) (width 0.3556) (layer F.Cu) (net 5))
 (segment (start 149.542 109.22) (end 151.892 109.22) (width 0.3556) (layer F.Cu) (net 5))
 (segment (start 151.892 109.22) (end 153.098 108.014) (width 0.3556) (layer F.Cu) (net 5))
 (segment (start 153.098 108.014) (end 161.29 108.014) (width 0.3556) (layer F.Cu) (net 5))
 (segment (start 161.29 108.014) (end 164.707 111.43) (width 0.3556) (layer F.Cu) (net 5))
 (segment (start 164.707 111.43) (end 164.707 115.316) (width 0.3556) (layer F.Cu) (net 5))
 (segment (start 164.707 115.316) (end 165.862 115.316) (width 0.3556) (layer F.Cu) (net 5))
 (segment (start 165.862 115.316) (end 166.434 115.888) (width 0.3556) (layer F.Cu) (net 5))
 (segment (start 166.434 115.888) (end 166.434 120.015) (width 0.3556) (layer F.Cu) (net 5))
 (segment (start 166.434 120.015) (end 165.672 120.777) (width 0.3556) (layer F.Cu) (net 5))
 (segment (start 165.672 120.777) (end 158.75 120.777) (width 0.3556) (layer F.Cu) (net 5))
 (segment (start 158.75 120.777) (end 158 120.027) (width 0.3556) (layer F.Cu) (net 5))
 (segment (start 158 120.027) (end 158 118.745) (width 0.3556) (layer F.Cu) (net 5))
 (segment (start 155.17 115.57) (end 157.29 115.57) (width 0.3556) (layer F.Cu) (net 5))
 (segment (start 157.29 115.57) (end 158 116.28) (width 0.3556) (layer F.Cu) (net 5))
 (segment (start 158 116.28) (end 158 118.745) (width 0.3556) (layer F.Cu) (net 5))
 (segment (start 145.3 103.505) (end 145.3 107.327) (width 0.3556) (layer F.Cu) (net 5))
 (segment (start 145.3 107.327) (end 145.542 107.569) (width 0.3556) (layer F.Cu) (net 5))
 (segment (start 145.542 107.569) (end 145.542 109.22) (width 0.3556) (layer F.Cu) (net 5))
 (segment (start 151.765 121.495) (end 151.765 117.475) (width 0.1524) (layer F.Cu) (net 2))
 (segment (start 151.765 117.475) (end 151.13 116.84) (width 0.1524) (layer F.Cu) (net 2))
 (segment (start 151.13 116.84) (end 151.13 115.57) (width 0.1524) (layer F.Cu) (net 2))
 (segment (start 161.745 117.86) (end 160.913 117.86) (width 0.1524) (layer F.Cu) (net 2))
 (segment (start 160.913 117.86) (end 160.528 117.475) (width 0.1524) (layer F.Cu) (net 2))
 (segment (start 160.528 117.475) (end 160.528 112.522) (width 0.1524) (layer F.Cu) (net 2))
 (segment (start 160.528 112.522) (end 159.766 111.76) (width 0.1524) (layer F.Cu) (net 2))
 (segment (start 159.766 111.76) (end 157.7 111.76) (width 0.1524) (layer F.Cu) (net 2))
 (segment (start 157.7 111.76) (end 154.686 111.76) (width 0.1524) (layer F.Cu) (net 2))
 (segment (start 154.686 111.76) (end 152.718 111.76) (width 0.1524) (layer B.Cu) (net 2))
 (segment (start 152.718 111.76) (end 151.702 111.76) (width 0.1524) (layer F.Cu) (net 2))
 (segment (start 151.702 111.76) (end 151.13 112.332) (width 0.1524) (layer F.Cu) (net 2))
 (segment (start 151.13 112.332) (end 151.13 115.57) (width 0.1524) (layer F.Cu) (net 2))
 (via (at 154.686 111.76) (size 0.508) (layers F.Cu B.Cu) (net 2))
 (via (at 152.718 111.76) (size 0.508) (layers F.Cu B.Cu) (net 2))
 (segment (start 153.035 121.495) (end 153.035 117.475) (width 0.1524) (layer F.Cu) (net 3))
 (segment (start 153.035 117.475) (end 153.67 116.84) (width 0.1524) (layer F.Cu) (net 3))
 (segment (start 153.67 116.84) (end 153.67 115.57) (width 0.1524) (layer F.Cu) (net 3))
 (segment (start 161.745 117.36) (end 161.745 110.056) (width 0.1524) (layer F.Cu) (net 3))
 (segment (start 161.745 110.056) (end 160.909 109.22) (width 0.1524) (layer F.Cu) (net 3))
 (segment (start 160.909 109.22) (end 157.7 109.22) (width 0.1524) (layer F.Cu) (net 3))
 (segment (start 153.67 115.57) (end 153.67 110.236) (width 0.1524) (layer F.Cu) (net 3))
 (segment (start 153.67 110.236) (end 154.686 109.22) (width 0.1524) (layer F.Cu) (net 3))
 (segment (start 154.686 109.22) (end 157.7 109.22) (width 0.1524) (layer F.Cu) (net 3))
 (segment (start 161.745 118.36) (end 160.722 118.36) (width 0.1524) (layer F.Cu) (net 6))
 (segment (start 160.722 118.36) (end 160.338 118.745) (width 0.1524) (layer F.Cu) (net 6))
 (segment (start 160.338 118.745) (end 159.5 118.745) (width 0.1524) (layer F.Cu) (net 6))
 (segment (start 147.1 106.68) (end 147.1 105.19) (width 0.1524) (layer F.Cu) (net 7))
 (segment (start 147.1 105.19) (end 146.8 104.89) (width 0.1524) (layer F.Cu) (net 7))
 (segment (start 146.8 104.89) (end 146.8 103.505) (width 0.1524) (layer F.Cu) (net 7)))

